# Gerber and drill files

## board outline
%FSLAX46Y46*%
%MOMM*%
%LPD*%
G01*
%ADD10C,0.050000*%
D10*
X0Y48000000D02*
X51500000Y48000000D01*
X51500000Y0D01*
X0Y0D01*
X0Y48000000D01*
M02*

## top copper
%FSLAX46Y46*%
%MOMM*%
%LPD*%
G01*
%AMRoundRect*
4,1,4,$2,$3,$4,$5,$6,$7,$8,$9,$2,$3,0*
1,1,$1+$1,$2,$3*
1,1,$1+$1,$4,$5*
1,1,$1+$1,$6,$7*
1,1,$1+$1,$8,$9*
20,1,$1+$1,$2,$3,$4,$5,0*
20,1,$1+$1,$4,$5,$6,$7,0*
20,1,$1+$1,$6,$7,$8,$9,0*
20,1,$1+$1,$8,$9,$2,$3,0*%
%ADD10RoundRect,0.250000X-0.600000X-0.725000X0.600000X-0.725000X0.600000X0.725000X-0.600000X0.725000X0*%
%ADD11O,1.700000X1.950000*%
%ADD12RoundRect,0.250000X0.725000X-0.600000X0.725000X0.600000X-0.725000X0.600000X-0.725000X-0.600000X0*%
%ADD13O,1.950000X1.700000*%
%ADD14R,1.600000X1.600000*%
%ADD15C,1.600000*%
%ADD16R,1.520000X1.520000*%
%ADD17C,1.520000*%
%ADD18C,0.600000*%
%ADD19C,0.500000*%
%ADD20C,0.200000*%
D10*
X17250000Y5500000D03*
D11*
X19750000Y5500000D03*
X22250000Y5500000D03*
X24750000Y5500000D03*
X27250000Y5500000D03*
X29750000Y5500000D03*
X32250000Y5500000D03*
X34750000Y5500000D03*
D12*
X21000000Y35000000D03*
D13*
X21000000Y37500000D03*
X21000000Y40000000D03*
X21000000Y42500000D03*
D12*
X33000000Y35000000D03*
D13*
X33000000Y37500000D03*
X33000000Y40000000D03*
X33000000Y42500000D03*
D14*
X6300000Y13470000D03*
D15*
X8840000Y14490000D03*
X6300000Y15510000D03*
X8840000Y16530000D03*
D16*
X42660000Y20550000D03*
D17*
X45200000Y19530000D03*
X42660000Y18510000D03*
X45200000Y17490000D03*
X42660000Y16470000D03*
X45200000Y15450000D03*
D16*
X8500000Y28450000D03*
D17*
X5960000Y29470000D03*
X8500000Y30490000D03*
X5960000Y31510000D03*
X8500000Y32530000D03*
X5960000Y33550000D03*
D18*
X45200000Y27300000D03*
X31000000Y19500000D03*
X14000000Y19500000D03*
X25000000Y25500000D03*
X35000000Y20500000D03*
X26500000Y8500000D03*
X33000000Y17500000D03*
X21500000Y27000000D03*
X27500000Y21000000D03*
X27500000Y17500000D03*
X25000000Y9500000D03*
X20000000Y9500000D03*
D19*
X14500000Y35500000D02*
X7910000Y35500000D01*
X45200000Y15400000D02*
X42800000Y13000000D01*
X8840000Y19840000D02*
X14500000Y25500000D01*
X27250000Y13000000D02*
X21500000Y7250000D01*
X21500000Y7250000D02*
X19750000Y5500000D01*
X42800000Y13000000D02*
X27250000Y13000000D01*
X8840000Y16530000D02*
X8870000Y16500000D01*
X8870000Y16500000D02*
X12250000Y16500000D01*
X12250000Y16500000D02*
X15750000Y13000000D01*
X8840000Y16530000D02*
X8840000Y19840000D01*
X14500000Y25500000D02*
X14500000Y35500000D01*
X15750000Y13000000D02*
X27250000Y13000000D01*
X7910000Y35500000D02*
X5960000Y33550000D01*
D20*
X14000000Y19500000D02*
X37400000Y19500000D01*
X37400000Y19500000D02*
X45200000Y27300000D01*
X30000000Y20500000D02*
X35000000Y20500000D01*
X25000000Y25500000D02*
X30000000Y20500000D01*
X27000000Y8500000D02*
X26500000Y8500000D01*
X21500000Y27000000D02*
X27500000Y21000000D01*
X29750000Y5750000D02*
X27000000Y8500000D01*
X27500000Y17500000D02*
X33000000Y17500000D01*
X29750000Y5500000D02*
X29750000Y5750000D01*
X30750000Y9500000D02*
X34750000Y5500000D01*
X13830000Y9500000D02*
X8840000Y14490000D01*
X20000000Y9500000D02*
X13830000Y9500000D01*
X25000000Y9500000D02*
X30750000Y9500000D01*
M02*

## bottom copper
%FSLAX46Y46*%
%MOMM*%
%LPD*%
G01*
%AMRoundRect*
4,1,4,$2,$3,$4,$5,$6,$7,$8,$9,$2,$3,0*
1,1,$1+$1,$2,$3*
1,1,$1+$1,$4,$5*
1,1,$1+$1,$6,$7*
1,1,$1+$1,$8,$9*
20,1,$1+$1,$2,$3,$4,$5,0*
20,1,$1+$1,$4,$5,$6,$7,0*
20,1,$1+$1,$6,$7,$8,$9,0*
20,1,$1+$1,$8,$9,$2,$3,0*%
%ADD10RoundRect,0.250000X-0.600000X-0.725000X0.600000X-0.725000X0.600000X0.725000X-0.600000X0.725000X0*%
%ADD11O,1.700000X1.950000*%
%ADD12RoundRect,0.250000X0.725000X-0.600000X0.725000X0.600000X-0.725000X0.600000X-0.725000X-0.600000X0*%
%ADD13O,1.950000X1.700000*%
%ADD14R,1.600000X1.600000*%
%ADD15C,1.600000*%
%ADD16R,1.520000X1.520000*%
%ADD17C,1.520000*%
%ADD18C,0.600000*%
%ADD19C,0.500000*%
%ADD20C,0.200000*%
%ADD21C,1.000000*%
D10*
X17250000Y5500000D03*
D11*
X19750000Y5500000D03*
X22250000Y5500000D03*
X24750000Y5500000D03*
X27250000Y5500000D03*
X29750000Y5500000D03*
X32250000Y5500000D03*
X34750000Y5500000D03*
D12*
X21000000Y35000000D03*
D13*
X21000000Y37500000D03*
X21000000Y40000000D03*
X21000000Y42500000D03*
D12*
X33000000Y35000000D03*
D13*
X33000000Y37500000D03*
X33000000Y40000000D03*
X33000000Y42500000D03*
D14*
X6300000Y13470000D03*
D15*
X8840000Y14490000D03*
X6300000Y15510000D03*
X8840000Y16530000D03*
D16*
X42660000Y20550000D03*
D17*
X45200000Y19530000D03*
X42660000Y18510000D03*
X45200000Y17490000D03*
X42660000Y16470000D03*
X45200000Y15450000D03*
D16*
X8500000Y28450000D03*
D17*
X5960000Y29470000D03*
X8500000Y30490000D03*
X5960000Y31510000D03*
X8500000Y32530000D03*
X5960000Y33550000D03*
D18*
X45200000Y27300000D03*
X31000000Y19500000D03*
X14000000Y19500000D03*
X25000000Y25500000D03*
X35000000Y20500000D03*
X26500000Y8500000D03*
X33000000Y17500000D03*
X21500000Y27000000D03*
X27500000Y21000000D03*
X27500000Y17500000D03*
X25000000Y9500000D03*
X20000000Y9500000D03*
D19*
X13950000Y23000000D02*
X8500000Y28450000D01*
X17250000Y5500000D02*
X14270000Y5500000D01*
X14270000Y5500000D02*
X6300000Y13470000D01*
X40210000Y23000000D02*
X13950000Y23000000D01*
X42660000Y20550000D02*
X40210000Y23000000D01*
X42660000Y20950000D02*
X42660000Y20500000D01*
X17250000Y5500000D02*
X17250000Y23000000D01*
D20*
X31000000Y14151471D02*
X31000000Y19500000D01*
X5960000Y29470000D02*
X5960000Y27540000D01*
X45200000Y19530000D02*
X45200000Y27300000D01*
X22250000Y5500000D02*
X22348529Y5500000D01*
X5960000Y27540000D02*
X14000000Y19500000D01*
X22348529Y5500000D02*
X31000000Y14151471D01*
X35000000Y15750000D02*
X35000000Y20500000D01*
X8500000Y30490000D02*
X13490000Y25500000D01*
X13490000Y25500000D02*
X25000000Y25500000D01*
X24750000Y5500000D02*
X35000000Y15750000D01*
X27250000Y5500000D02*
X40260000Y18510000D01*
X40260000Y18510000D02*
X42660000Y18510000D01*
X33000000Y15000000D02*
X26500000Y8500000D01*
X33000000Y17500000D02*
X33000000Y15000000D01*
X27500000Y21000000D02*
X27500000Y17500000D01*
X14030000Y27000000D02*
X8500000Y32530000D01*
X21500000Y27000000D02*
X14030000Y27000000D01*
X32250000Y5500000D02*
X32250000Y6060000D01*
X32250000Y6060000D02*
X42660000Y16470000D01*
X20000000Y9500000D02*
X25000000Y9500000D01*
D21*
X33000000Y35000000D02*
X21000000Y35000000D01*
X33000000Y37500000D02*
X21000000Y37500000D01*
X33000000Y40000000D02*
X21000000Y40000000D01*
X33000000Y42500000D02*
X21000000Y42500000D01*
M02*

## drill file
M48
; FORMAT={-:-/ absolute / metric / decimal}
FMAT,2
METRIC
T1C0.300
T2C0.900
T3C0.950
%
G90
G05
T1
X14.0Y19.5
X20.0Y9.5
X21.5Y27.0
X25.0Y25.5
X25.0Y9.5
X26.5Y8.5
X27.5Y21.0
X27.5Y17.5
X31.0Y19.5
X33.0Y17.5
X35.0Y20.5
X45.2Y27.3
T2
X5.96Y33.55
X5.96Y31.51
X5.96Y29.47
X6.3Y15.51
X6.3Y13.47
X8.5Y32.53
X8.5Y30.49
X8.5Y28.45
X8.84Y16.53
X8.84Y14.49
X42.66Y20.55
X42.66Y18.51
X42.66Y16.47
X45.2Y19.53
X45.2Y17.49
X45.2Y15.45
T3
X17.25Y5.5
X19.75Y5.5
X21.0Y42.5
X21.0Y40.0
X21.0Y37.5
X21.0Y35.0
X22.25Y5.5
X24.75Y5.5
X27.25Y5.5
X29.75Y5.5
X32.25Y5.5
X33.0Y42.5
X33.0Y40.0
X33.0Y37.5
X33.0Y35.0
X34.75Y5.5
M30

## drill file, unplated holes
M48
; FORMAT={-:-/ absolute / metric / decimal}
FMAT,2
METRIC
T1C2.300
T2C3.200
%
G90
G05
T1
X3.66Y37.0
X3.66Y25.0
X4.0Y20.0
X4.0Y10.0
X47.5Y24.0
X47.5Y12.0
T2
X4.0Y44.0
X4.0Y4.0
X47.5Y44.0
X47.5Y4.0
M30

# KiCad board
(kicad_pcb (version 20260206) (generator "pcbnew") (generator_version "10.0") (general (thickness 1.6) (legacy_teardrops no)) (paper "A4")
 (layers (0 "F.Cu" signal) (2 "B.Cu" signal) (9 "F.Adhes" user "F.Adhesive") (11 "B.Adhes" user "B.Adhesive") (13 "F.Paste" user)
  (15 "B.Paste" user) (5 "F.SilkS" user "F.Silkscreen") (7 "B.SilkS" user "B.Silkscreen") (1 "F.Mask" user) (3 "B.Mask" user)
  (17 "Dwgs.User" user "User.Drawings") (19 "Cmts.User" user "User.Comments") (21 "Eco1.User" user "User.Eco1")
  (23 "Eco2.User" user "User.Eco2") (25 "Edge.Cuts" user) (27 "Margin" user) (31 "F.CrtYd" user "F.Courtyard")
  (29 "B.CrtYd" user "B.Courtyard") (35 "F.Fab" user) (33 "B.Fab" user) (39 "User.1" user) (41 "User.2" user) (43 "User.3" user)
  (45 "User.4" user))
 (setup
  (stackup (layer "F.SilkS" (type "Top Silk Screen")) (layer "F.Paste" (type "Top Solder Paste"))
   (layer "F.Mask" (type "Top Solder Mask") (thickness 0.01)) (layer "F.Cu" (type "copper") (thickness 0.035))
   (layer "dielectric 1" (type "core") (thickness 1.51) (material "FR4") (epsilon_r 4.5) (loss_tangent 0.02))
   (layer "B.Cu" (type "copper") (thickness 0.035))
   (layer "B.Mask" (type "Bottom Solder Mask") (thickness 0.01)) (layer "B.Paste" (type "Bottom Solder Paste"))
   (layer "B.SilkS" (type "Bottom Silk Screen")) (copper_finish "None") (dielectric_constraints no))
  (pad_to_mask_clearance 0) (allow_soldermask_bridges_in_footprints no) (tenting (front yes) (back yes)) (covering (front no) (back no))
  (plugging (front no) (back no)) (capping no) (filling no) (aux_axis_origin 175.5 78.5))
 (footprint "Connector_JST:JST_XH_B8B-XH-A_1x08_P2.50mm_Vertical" (layer "F.Cu") (at 192.75 73)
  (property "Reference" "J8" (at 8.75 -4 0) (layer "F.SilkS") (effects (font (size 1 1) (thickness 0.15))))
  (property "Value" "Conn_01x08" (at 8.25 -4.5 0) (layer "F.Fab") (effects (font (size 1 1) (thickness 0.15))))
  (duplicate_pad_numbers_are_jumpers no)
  (pad "1" thru_hole roundrect (at 0 0) (size 1.7 1.95) (drill 0.95) (layers "*.Cu" "*.Mask") (remove_unused_layers no)
   (roundrect_rratio 0.147059) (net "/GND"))
  (pad "2" thru_hole oval (at 2.5 0) (size 1.7 1.95) (drill 0.95) (layers "*.Cu" "*.Mask") (remove_unused_layers no) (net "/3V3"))
  (pad "3" thru_hole oval (at 5 0) (size 1.7 1.95) (drill 0.95) (layers "*.Cu" "*.Mask") (remove_unused_layers no) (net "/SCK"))
  (pad "4" thru_hole oval (at 7.5 0) (size 1.7 1.95) (drill 0.95) (layers "*.Cu" "*.Mask") (remove_unused_layers no) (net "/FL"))
  (pad "5" thru_hole oval (at 10 0) (size 1.7 1.95) (drill 0.95) (layers "*.Cu" "*.Mask") (remove_unused_layers no) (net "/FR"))
  (pad "6" thru_hole oval (at 12.5 0) (size 1.7 1.95) (drill 0.95) (layers "*.Cu" "*.Mask") (remove_unused_layers no) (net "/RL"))
  (pad "7" thru_hole oval (at 15 0) (size 1.7 1.95) (drill 0.95) (layers "*.Cu" "*.Mask") (remove_unused_layers no) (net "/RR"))
  (pad "8" thru_hole oval (at 17.5 0) (size 1.7 1.95) (drill 0.95) (layers "*.Cu" "*.Mask") (remove_unused_layers no) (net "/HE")))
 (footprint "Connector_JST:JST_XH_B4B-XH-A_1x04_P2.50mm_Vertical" (layer "F.Cu") (at 196.5 43.5 90)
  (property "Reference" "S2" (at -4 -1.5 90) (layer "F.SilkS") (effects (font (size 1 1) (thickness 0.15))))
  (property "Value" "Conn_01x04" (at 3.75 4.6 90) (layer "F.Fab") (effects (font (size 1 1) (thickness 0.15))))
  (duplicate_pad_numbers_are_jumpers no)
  (pad "1" thru_hole roundrect (at 0 0 90) (size 1.7 1.95) (drill 0.95) (layers "*.Cu" "*.Mask") (remove_unused_layers no)
   (roundrect_rratio 0.147059) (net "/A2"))
  (pad "2" thru_hole oval (at 2.5 0 90) (size 1.7 1.95) (drill 0.95) (layers "*.Cu" "*.Mask") (remove_unused_layers no) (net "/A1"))
  (pad "3" thru_hole oval (at 5 0 90) (size 1.7 1.95) (drill 0.95) (layers "*.Cu" "*.Mask") (remove_unused_layers no) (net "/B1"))
  (pad "4" thru_hole oval (at 7.5 0 90) (size 1.7 1.95) (drill 0.95) (layers "*.Cu" "*.Mask") (remove_unused_layers no) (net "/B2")))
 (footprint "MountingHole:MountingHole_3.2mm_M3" (layer "F.Cu") (at 223 34.5)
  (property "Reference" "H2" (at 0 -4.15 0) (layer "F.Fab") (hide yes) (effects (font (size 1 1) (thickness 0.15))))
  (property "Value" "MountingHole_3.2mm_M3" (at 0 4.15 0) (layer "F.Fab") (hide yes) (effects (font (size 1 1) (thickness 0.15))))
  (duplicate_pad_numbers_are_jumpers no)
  (pad "" np_thru_hole circle (at 0 0) (size 3.2 3.2) (drill 3.2) (layers "*.Cu" "*.Mask")))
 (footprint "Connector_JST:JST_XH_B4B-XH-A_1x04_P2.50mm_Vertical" (layer "F.Cu") (at 208.5 43.5 90)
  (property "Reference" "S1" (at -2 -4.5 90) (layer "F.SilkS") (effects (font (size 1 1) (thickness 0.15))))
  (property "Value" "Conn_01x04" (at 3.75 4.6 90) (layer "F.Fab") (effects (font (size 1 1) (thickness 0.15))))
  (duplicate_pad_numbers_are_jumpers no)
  (pad "1" thru_hole roundrect (at 0 0 90) (size 1.7 1.95) (drill 0.95) (layers "*.Cu" "*.Mask") (remove_unused_layers no)
   (roundrect_rratio 0.147059) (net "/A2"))
  (pad "2" thru_hole oval (at 2.5 0 90) (size 1.7 1.95) (drill 0.95) (layers "*.Cu" "*.Mask") (remove_unused_layers no) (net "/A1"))
  (pad "3" thru_hole oval (at 5 0 90) (size 1.7 1.95) (drill 0.95) (layers "*.Cu" "*.Mask") (remove_unused_layers no) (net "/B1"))
  (pad "4" thru_hole oval (at 7.5 0 90) (size 1.7 1.95) (drill 0.95) (layers "*.Cu" "*.Mask") (remove_unused_layers no) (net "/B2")))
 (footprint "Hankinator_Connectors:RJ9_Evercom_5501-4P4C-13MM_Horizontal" (layer "F.Cu") (at 179.5 63.5 -90)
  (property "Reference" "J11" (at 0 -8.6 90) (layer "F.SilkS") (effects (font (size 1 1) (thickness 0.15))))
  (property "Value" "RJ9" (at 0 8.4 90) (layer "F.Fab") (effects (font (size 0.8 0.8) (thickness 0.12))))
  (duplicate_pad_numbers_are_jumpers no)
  (pad "" np_thru_hole circle (at -5 0 270) (size 2.3 2.3) (drill 2.3) (layers "*.Cu" "*.Mask"))
  (pad "" np_thru_hole circle (at 5 0 270) (size 2.3 2.3) (drill 2.3) (layers "*.Cu" "*.Mask"))
  (pad "1" thru_hole rect (at 1.53 -2.3 270) (size 1.6 1.6) (drill 0.9) (layers "*.Cu" "*.Mask") (remove_unused_layers no) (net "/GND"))
  (pad "2" thru_hole circle (at 0.51 -4.84 270) (size 1.6 1.6) (drill 0.9) (layers "*.Cu" "*.Mask") (remove_unused_layers no) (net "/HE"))
  (pad "3" thru_hole circle (at -0.51 -2.3 270) (size 1.6 1.6) (drill 0.9) (layers "*.Cu" "*.Mask") (remove_unused_layers no)
   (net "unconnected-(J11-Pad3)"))
  (pad "4" thru_hole circle (at -1.53 -4.84 270) (size 1.6 1.6) (drill 0.9) (layers "*.Cu" "*.Mask") (remove_unused_layers no) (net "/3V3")))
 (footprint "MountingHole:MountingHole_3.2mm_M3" (layer "F.Cu") (at 179.5 34.5)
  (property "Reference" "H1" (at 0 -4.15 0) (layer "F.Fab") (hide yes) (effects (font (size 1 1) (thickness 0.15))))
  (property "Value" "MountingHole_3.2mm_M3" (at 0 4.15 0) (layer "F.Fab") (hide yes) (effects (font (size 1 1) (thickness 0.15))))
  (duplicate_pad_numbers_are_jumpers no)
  (pad "" np_thru_hole circle (at 0 0) (size 3.2 3.2) (drill 3.2) (layers "*.Cu" "*.Mask")))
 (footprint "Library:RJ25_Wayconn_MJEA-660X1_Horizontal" (layer "F.Cu") (at 218.16 57.95 90)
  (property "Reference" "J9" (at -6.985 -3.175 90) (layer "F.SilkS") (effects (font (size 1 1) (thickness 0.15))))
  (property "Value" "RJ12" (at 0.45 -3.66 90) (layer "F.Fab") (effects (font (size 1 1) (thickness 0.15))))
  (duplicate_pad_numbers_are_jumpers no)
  (pad "" np_thru_hole circle (at -8.55 4.84 90) (size 2.3 2.3) (drill 2.3) (layers "*.Cu" "*.Mask"))
  (pad "" np_thru_hole circle (at 3.45 4.84 90) (size 2.3 2.3) (drill 2.3) (layers "*.Cu" "*.Mask"))
  (pad "1" thru_hole rect (at 0 0 90) (size 1.52 1.52) (drill 0.9) (layers "*.Cu" "*.Mask") (remove_unused_layers no) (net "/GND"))
  (pad "2" thru_hole circle (at -1.02 2.54 90) (size 1.52 1.52) (drill 0.9) (layers "*.Cu" "*.Mask") (remove_unused_layers no) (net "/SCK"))
  (pad "3" thru_hole circle (at -2.04 0 90) (size 1.52 1.52) (drill 0.9) (layers "*.Cu" "*.Mask") (remove_unused_layers no) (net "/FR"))
  (pad "4" thru_hole circle (at -3.06 2.54 90) (size 1.52 1.52) (drill 0.9) (layers "*.Cu" "*.Mask") (remove_unused_layers no)
   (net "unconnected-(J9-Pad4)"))
  (pad "5" thru_hole circle (at -4.08 0 90) (size 1.52 1.52) (drill 0.9) (layers "*.Cu" "*.Mask") (remove_unused_layers no) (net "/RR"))
  (pad "6" thru_hole circle (at -5.1 2.54 90) (size 1.52 1.52) (drill 0.9) (layers "*.Cu" "*.Mask") (remove_unused_layers no) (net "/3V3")))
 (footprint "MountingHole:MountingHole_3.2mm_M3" (layer "F.Cu") (at 223 74.5)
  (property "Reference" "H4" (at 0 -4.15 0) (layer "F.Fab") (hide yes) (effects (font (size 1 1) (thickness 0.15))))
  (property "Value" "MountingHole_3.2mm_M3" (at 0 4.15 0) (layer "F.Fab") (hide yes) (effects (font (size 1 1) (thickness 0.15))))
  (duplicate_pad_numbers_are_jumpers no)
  (pad "" np_thru_hole circle (at 0 0) (size 3.2 3.2) (drill 3.2) (layers "*.Cu" "*.Mask")))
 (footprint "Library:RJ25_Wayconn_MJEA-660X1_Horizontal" (layer "F.Cu") (at 184 50.05 -90)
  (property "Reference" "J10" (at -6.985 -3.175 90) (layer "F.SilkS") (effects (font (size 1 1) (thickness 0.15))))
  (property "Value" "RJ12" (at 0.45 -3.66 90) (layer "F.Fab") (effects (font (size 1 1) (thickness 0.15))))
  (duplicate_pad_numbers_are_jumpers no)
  (pad "" np_thru_hole circle (at -8.55 4.84 270) (size 2.3 2.3) (drill 2.3) (layers "*.Cu" "*.Mask"))
  (pad "" np_thru_hole circle (at 3.45 4.84 270) (size 2.3 2.3) (drill 2.3) (layers "*.Cu" "*.Mask"))
  (pad "1" thru_hole rect (at 0 0 270) (size 1.52 1.52) (drill 0.9) (layers "*.Cu" "*.Mask") (remove_unused_layers no) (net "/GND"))
  (pad "2" thru_hole circle (at -1.02 2.54 270) (size 1.52 1.52) (drill 0.9) (layers "*.Cu" "*.Mask") (remove_unused_layers no) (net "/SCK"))
  (pad "3" thru_hole circle (at -2.04 0 270) (size 1.52 1.52) (drill 0.9) (layers "*.Cu" "*.Mask") (remove_unused_layers no) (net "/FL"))
  (pad "4" thru_hole circle (at -3.06 2.54 270) (size 1.52 1.52) (drill 0.9) (layers "*.Cu" "*.Mask") (remove_unused_layers no)
   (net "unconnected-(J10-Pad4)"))
  (pad "5" thru_hole circle (at -4.08 0 270) (size 1.52 1.52) (drill 0.9) (layers "*.Cu" "*.Mask") (remove_unused_layers no) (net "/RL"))
  (pad "6" thru_hole circle (at -5.1 2.54 270) (size 1.52 1.52) (drill 0.9) (layers "*.Cu" "*.Mask") (remove_unused_layers no) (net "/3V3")))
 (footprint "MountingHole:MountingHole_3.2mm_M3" (layer "F.Cu") (at 179.5 74.5)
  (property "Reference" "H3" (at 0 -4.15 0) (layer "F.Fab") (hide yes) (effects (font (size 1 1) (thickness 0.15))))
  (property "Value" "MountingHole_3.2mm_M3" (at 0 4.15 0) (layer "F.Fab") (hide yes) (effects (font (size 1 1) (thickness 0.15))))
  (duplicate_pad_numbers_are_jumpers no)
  (pad "" np_thru_hole circle (at 0 0) (size 3.2 3.2) (drill 3.2) (layers "*.Cu" "*.Mask")))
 (gr_rect (start 175.5 30.5) (end 227 78.5) (stroke (width 0.05) (type default)) (fill no) (layer "Edge.Cuts"))
 (segment (start 189.45 55.5) (end 184 50.05) (width 0.5) (layer "B.Cu") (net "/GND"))
 (segment (start 192.75 73) (end 189.77 73) (width 0.5) (layer "B.Cu") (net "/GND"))
 (segment (start 189.77 73) (end 181.8 65.03) (width 0.5) (layer "B.Cu") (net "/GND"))
 (segment (start 215.71 55.5) (end 189.45 55.5) (width 0.5) (layer "B.Cu") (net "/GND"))
 (segment (start 218.16 57.95) (end 215.71 55.5) (width 0.5) (layer "B.Cu") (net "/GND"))
 (segment (start 218.16 57.55) (end 218.16 58) (width 0.5) (layer "B.Cu") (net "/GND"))
 (segment (start 192.75 73) (end 192.75 55.5) (width 0.5) (layer "B.Cu") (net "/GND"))
 (segment (start 190 43) (end 183.41 43) (width 0.5) (layer "F.Cu") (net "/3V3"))
 (segment (start 220.7 63.1) (end 218.3 65.5) (width 0.5) (layer "F.Cu") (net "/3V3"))
 (segment (start 184.34 58.66) (end 190 53) (width 0.5) (layer "F.Cu") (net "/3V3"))
 (segment (start 202.75 65.5) (end 197 71.25) (width 0.5) (layer "F.Cu") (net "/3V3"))
 (segment (start 197 71.25) (end 195.25 73) (width 0.5) (layer "F.Cu") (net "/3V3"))
 (segment (start 218.3 65.5) (end 202.75 65.5) (width 0.5) (layer "F.Cu") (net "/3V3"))
 (segment (start 184.34 61.97) (end 184.37 62) (width 0.5) (layer "F.Cu") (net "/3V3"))
 (segment (start 184.37 62) (end 187.75 62) (width 0.5) (layer "F.Cu") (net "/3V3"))
 (segment (start 187.75 62) (end 191.25 65.5) (width 0.5) (layer "F.Cu") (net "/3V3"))
 (segment (start 184.34 61.97) (end 184.34 58.66) (width 0.5) (layer "F.Cu") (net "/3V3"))
 (segment (start 190 53) (end 190 43) (width 0.5) (layer "F.Cu") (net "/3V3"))
 (segment (start 191.25 65.5) (end 202.75 65.5) (width 0.5) (layer "F.Cu") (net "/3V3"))
 (segment (start 183.41 43) (end 181.46 44.95) (width 0.5) (layer "F.Cu") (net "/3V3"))
 (segment (start 189.5 59) (end 212.9 59) (width 0.2) (layer "F.Cu") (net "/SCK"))
 (segment (start 212.9 59) (end 220.7 51.2) (width 0.2) (layer "F.Cu") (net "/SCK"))
 (via (at 220.7 51.2) (size 0.6) (drill 0.3) (layers "F.Cu" "B.Cu") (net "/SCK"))
 (via (at 206.5 59) (size 0.6) (drill 0.3) (layers "F.Cu" "B.Cu") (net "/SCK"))
 (via (at 189.5 59) (size 0.6) (drill 0.3) (layers "F.Cu" "B.Cu") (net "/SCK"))
 (segment (start 206.5 64.348529) (end 206.5 59) (width 0.2) (layer "B.Cu") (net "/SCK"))
 (segment (start 181.46 49.03) (end 181.46 50.96) (width 0.2) (layer "B.Cu") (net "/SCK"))
 (segment (start 220.7 58.97) (end 220.7 51.2) (width 0.2) (layer "B.Cu") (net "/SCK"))
 (segment (start 197.75 73) (end 197.848529 73) (width 0.2) (layer "B.Cu") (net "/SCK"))
 (segment (start 181.46 50.96) (end 189.5 59) (width 0.2) (layer "B.Cu") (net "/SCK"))
 (segment (start 197.848529 73) (end 206.5 64.348529) (width 0.2) (layer "B.Cu") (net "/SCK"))
 (segment (start 205.5 58) (end 210.5 58) (width 0.2) (layer "F.Cu") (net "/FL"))
 (segment (start 200.5 53) (end 205.5 58) (width 0.2) (layer "F.Cu") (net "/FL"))
 (via (at 200.5 53) (size 0.6) (drill 0.3) (layers "F.Cu" "B.Cu") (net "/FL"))
 (via (at 210.5 58) (size 0.6) (drill 0.3) (layers "F.Cu" "B.Cu") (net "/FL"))
 (segment (start 210.5 62.75) (end 210.5 58) (width 0.2) (layer "B.Cu") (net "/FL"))
 (segment (start 184 48.01) (end 188.99 53) (width 0.2) (layer "B.Cu") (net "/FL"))
 (segment (start 188.99 53) (end 200.5 53) (width 0.2) (layer "B.Cu") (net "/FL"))
 (segment (start 200.25 73) (end 210.5 62.75) (width 0.2) (layer "B.Cu") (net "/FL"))
 (segment (start 202.75 73) (end 215.76 59.99) (width 0.2) (layer "B.Cu") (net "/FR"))
 (segment (start 215.76 59.99) (end 218.16 59.99) (width 0.2) (layer "B.Cu") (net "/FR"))
 (segment (start 202.5 70) (end 202 70) (width 0.2) (layer "F.Cu") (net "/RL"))
 (segment (start 197 51.5) (end 203 57.5) (width 0.2) (layer "F.Cu") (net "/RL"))
 (segment (start 205.25 72.75) (end 202.5 70) (width 0.2) (layer "F.Cu") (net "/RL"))
 (segment (start 203 61) (end 208.5 61) (width 0.2) (layer "F.Cu") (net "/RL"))
 (segment (start 205.25 73) (end 205.25 72.75) (width 0.2) (layer "F.Cu") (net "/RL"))
 (via (at 202 70) (size 0.6) (drill 0.3) (layers "F.Cu" "B.Cu") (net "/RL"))
 (via (at 208.5 61) (size 0.6) (drill 0.3) (layers "F.Cu" "B.Cu") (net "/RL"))
 (via (at 197 51.5) (size 0.6) (drill 0.3) (layers "F.Cu" "B.Cu") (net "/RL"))
 (via (at 203 57.5) (size 0.6) (drill 0.3) (layers "F.Cu" "B.Cu") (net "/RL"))
 (via (at 203 61) (size 0.6) (drill 0.3) (layers "F.Cu" "B.Cu") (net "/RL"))
 (segment (start 208.5 63.5) (end 202 70) (width 0.2) (layer "B.Cu") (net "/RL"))
 (segment (start 208.5 61) (end 208.5 63.5) (width 0.2) (layer "B.Cu") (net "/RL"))
 (segment (start 203 57.5) (end 203 61) (width 0.2) (layer "B.Cu") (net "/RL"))
 (segment (start 189.53 51.5) (end 184 45.97) (width 0.2) (layer "B.Cu") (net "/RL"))
 (segment (start 197 51.5) (end 189.53 51.5) (width 0.2) (layer "B.Cu") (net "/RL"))
 (segment (start 207.75 73) (end 207.75 72.44) (width 0.2) (layer "B.Cu") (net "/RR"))
 (segment (start 207.75 72.44) (end 218.16 62.03) (width 0.2) (layer "B.Cu") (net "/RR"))
 (segment (start 206.25 69) (end 210.25 73) (width 0.2) (layer "F.Cu") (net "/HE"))
 (segment (start 189.33 69) (end 184.34 64.01) (width 0.2) (layer "F.Cu") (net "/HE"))
 (segment (start 195.5 69) (end 189.33 69) (width 0.2) (layer "F.Cu") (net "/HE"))
 (segment (start 200.5 69) (end 206.25 69) (width 0.2) (layer "F.Cu") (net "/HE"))
 (via (at 200.5 69) (size 0.6) (drill 0.3) (layers "F.Cu" "B.Cu") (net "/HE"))
 (via (at 195.5 69) (size 0.6) (drill 0.3) (layers "F.Cu" "B.Cu") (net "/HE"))
 (segment (start 195.5 69) (end 200.5 69) (width 0.2) (layer "B.Cu") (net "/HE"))
 (segment (start 208.5 43.5) (end 196.5 43.5) (width 1) (layer "B.Cu") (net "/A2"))
 (segment (start 208.5 41) (end 196.5 41) (width 1) (layer "B.Cu") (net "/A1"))
 (segment (start 208.5 38.5) (end 196.5 38.5) (width 1) (layer "B.Cu") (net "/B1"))
 (segment (start 208.5 36) (end 196.5 36) (width 1) (layer "B.Cu") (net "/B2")))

